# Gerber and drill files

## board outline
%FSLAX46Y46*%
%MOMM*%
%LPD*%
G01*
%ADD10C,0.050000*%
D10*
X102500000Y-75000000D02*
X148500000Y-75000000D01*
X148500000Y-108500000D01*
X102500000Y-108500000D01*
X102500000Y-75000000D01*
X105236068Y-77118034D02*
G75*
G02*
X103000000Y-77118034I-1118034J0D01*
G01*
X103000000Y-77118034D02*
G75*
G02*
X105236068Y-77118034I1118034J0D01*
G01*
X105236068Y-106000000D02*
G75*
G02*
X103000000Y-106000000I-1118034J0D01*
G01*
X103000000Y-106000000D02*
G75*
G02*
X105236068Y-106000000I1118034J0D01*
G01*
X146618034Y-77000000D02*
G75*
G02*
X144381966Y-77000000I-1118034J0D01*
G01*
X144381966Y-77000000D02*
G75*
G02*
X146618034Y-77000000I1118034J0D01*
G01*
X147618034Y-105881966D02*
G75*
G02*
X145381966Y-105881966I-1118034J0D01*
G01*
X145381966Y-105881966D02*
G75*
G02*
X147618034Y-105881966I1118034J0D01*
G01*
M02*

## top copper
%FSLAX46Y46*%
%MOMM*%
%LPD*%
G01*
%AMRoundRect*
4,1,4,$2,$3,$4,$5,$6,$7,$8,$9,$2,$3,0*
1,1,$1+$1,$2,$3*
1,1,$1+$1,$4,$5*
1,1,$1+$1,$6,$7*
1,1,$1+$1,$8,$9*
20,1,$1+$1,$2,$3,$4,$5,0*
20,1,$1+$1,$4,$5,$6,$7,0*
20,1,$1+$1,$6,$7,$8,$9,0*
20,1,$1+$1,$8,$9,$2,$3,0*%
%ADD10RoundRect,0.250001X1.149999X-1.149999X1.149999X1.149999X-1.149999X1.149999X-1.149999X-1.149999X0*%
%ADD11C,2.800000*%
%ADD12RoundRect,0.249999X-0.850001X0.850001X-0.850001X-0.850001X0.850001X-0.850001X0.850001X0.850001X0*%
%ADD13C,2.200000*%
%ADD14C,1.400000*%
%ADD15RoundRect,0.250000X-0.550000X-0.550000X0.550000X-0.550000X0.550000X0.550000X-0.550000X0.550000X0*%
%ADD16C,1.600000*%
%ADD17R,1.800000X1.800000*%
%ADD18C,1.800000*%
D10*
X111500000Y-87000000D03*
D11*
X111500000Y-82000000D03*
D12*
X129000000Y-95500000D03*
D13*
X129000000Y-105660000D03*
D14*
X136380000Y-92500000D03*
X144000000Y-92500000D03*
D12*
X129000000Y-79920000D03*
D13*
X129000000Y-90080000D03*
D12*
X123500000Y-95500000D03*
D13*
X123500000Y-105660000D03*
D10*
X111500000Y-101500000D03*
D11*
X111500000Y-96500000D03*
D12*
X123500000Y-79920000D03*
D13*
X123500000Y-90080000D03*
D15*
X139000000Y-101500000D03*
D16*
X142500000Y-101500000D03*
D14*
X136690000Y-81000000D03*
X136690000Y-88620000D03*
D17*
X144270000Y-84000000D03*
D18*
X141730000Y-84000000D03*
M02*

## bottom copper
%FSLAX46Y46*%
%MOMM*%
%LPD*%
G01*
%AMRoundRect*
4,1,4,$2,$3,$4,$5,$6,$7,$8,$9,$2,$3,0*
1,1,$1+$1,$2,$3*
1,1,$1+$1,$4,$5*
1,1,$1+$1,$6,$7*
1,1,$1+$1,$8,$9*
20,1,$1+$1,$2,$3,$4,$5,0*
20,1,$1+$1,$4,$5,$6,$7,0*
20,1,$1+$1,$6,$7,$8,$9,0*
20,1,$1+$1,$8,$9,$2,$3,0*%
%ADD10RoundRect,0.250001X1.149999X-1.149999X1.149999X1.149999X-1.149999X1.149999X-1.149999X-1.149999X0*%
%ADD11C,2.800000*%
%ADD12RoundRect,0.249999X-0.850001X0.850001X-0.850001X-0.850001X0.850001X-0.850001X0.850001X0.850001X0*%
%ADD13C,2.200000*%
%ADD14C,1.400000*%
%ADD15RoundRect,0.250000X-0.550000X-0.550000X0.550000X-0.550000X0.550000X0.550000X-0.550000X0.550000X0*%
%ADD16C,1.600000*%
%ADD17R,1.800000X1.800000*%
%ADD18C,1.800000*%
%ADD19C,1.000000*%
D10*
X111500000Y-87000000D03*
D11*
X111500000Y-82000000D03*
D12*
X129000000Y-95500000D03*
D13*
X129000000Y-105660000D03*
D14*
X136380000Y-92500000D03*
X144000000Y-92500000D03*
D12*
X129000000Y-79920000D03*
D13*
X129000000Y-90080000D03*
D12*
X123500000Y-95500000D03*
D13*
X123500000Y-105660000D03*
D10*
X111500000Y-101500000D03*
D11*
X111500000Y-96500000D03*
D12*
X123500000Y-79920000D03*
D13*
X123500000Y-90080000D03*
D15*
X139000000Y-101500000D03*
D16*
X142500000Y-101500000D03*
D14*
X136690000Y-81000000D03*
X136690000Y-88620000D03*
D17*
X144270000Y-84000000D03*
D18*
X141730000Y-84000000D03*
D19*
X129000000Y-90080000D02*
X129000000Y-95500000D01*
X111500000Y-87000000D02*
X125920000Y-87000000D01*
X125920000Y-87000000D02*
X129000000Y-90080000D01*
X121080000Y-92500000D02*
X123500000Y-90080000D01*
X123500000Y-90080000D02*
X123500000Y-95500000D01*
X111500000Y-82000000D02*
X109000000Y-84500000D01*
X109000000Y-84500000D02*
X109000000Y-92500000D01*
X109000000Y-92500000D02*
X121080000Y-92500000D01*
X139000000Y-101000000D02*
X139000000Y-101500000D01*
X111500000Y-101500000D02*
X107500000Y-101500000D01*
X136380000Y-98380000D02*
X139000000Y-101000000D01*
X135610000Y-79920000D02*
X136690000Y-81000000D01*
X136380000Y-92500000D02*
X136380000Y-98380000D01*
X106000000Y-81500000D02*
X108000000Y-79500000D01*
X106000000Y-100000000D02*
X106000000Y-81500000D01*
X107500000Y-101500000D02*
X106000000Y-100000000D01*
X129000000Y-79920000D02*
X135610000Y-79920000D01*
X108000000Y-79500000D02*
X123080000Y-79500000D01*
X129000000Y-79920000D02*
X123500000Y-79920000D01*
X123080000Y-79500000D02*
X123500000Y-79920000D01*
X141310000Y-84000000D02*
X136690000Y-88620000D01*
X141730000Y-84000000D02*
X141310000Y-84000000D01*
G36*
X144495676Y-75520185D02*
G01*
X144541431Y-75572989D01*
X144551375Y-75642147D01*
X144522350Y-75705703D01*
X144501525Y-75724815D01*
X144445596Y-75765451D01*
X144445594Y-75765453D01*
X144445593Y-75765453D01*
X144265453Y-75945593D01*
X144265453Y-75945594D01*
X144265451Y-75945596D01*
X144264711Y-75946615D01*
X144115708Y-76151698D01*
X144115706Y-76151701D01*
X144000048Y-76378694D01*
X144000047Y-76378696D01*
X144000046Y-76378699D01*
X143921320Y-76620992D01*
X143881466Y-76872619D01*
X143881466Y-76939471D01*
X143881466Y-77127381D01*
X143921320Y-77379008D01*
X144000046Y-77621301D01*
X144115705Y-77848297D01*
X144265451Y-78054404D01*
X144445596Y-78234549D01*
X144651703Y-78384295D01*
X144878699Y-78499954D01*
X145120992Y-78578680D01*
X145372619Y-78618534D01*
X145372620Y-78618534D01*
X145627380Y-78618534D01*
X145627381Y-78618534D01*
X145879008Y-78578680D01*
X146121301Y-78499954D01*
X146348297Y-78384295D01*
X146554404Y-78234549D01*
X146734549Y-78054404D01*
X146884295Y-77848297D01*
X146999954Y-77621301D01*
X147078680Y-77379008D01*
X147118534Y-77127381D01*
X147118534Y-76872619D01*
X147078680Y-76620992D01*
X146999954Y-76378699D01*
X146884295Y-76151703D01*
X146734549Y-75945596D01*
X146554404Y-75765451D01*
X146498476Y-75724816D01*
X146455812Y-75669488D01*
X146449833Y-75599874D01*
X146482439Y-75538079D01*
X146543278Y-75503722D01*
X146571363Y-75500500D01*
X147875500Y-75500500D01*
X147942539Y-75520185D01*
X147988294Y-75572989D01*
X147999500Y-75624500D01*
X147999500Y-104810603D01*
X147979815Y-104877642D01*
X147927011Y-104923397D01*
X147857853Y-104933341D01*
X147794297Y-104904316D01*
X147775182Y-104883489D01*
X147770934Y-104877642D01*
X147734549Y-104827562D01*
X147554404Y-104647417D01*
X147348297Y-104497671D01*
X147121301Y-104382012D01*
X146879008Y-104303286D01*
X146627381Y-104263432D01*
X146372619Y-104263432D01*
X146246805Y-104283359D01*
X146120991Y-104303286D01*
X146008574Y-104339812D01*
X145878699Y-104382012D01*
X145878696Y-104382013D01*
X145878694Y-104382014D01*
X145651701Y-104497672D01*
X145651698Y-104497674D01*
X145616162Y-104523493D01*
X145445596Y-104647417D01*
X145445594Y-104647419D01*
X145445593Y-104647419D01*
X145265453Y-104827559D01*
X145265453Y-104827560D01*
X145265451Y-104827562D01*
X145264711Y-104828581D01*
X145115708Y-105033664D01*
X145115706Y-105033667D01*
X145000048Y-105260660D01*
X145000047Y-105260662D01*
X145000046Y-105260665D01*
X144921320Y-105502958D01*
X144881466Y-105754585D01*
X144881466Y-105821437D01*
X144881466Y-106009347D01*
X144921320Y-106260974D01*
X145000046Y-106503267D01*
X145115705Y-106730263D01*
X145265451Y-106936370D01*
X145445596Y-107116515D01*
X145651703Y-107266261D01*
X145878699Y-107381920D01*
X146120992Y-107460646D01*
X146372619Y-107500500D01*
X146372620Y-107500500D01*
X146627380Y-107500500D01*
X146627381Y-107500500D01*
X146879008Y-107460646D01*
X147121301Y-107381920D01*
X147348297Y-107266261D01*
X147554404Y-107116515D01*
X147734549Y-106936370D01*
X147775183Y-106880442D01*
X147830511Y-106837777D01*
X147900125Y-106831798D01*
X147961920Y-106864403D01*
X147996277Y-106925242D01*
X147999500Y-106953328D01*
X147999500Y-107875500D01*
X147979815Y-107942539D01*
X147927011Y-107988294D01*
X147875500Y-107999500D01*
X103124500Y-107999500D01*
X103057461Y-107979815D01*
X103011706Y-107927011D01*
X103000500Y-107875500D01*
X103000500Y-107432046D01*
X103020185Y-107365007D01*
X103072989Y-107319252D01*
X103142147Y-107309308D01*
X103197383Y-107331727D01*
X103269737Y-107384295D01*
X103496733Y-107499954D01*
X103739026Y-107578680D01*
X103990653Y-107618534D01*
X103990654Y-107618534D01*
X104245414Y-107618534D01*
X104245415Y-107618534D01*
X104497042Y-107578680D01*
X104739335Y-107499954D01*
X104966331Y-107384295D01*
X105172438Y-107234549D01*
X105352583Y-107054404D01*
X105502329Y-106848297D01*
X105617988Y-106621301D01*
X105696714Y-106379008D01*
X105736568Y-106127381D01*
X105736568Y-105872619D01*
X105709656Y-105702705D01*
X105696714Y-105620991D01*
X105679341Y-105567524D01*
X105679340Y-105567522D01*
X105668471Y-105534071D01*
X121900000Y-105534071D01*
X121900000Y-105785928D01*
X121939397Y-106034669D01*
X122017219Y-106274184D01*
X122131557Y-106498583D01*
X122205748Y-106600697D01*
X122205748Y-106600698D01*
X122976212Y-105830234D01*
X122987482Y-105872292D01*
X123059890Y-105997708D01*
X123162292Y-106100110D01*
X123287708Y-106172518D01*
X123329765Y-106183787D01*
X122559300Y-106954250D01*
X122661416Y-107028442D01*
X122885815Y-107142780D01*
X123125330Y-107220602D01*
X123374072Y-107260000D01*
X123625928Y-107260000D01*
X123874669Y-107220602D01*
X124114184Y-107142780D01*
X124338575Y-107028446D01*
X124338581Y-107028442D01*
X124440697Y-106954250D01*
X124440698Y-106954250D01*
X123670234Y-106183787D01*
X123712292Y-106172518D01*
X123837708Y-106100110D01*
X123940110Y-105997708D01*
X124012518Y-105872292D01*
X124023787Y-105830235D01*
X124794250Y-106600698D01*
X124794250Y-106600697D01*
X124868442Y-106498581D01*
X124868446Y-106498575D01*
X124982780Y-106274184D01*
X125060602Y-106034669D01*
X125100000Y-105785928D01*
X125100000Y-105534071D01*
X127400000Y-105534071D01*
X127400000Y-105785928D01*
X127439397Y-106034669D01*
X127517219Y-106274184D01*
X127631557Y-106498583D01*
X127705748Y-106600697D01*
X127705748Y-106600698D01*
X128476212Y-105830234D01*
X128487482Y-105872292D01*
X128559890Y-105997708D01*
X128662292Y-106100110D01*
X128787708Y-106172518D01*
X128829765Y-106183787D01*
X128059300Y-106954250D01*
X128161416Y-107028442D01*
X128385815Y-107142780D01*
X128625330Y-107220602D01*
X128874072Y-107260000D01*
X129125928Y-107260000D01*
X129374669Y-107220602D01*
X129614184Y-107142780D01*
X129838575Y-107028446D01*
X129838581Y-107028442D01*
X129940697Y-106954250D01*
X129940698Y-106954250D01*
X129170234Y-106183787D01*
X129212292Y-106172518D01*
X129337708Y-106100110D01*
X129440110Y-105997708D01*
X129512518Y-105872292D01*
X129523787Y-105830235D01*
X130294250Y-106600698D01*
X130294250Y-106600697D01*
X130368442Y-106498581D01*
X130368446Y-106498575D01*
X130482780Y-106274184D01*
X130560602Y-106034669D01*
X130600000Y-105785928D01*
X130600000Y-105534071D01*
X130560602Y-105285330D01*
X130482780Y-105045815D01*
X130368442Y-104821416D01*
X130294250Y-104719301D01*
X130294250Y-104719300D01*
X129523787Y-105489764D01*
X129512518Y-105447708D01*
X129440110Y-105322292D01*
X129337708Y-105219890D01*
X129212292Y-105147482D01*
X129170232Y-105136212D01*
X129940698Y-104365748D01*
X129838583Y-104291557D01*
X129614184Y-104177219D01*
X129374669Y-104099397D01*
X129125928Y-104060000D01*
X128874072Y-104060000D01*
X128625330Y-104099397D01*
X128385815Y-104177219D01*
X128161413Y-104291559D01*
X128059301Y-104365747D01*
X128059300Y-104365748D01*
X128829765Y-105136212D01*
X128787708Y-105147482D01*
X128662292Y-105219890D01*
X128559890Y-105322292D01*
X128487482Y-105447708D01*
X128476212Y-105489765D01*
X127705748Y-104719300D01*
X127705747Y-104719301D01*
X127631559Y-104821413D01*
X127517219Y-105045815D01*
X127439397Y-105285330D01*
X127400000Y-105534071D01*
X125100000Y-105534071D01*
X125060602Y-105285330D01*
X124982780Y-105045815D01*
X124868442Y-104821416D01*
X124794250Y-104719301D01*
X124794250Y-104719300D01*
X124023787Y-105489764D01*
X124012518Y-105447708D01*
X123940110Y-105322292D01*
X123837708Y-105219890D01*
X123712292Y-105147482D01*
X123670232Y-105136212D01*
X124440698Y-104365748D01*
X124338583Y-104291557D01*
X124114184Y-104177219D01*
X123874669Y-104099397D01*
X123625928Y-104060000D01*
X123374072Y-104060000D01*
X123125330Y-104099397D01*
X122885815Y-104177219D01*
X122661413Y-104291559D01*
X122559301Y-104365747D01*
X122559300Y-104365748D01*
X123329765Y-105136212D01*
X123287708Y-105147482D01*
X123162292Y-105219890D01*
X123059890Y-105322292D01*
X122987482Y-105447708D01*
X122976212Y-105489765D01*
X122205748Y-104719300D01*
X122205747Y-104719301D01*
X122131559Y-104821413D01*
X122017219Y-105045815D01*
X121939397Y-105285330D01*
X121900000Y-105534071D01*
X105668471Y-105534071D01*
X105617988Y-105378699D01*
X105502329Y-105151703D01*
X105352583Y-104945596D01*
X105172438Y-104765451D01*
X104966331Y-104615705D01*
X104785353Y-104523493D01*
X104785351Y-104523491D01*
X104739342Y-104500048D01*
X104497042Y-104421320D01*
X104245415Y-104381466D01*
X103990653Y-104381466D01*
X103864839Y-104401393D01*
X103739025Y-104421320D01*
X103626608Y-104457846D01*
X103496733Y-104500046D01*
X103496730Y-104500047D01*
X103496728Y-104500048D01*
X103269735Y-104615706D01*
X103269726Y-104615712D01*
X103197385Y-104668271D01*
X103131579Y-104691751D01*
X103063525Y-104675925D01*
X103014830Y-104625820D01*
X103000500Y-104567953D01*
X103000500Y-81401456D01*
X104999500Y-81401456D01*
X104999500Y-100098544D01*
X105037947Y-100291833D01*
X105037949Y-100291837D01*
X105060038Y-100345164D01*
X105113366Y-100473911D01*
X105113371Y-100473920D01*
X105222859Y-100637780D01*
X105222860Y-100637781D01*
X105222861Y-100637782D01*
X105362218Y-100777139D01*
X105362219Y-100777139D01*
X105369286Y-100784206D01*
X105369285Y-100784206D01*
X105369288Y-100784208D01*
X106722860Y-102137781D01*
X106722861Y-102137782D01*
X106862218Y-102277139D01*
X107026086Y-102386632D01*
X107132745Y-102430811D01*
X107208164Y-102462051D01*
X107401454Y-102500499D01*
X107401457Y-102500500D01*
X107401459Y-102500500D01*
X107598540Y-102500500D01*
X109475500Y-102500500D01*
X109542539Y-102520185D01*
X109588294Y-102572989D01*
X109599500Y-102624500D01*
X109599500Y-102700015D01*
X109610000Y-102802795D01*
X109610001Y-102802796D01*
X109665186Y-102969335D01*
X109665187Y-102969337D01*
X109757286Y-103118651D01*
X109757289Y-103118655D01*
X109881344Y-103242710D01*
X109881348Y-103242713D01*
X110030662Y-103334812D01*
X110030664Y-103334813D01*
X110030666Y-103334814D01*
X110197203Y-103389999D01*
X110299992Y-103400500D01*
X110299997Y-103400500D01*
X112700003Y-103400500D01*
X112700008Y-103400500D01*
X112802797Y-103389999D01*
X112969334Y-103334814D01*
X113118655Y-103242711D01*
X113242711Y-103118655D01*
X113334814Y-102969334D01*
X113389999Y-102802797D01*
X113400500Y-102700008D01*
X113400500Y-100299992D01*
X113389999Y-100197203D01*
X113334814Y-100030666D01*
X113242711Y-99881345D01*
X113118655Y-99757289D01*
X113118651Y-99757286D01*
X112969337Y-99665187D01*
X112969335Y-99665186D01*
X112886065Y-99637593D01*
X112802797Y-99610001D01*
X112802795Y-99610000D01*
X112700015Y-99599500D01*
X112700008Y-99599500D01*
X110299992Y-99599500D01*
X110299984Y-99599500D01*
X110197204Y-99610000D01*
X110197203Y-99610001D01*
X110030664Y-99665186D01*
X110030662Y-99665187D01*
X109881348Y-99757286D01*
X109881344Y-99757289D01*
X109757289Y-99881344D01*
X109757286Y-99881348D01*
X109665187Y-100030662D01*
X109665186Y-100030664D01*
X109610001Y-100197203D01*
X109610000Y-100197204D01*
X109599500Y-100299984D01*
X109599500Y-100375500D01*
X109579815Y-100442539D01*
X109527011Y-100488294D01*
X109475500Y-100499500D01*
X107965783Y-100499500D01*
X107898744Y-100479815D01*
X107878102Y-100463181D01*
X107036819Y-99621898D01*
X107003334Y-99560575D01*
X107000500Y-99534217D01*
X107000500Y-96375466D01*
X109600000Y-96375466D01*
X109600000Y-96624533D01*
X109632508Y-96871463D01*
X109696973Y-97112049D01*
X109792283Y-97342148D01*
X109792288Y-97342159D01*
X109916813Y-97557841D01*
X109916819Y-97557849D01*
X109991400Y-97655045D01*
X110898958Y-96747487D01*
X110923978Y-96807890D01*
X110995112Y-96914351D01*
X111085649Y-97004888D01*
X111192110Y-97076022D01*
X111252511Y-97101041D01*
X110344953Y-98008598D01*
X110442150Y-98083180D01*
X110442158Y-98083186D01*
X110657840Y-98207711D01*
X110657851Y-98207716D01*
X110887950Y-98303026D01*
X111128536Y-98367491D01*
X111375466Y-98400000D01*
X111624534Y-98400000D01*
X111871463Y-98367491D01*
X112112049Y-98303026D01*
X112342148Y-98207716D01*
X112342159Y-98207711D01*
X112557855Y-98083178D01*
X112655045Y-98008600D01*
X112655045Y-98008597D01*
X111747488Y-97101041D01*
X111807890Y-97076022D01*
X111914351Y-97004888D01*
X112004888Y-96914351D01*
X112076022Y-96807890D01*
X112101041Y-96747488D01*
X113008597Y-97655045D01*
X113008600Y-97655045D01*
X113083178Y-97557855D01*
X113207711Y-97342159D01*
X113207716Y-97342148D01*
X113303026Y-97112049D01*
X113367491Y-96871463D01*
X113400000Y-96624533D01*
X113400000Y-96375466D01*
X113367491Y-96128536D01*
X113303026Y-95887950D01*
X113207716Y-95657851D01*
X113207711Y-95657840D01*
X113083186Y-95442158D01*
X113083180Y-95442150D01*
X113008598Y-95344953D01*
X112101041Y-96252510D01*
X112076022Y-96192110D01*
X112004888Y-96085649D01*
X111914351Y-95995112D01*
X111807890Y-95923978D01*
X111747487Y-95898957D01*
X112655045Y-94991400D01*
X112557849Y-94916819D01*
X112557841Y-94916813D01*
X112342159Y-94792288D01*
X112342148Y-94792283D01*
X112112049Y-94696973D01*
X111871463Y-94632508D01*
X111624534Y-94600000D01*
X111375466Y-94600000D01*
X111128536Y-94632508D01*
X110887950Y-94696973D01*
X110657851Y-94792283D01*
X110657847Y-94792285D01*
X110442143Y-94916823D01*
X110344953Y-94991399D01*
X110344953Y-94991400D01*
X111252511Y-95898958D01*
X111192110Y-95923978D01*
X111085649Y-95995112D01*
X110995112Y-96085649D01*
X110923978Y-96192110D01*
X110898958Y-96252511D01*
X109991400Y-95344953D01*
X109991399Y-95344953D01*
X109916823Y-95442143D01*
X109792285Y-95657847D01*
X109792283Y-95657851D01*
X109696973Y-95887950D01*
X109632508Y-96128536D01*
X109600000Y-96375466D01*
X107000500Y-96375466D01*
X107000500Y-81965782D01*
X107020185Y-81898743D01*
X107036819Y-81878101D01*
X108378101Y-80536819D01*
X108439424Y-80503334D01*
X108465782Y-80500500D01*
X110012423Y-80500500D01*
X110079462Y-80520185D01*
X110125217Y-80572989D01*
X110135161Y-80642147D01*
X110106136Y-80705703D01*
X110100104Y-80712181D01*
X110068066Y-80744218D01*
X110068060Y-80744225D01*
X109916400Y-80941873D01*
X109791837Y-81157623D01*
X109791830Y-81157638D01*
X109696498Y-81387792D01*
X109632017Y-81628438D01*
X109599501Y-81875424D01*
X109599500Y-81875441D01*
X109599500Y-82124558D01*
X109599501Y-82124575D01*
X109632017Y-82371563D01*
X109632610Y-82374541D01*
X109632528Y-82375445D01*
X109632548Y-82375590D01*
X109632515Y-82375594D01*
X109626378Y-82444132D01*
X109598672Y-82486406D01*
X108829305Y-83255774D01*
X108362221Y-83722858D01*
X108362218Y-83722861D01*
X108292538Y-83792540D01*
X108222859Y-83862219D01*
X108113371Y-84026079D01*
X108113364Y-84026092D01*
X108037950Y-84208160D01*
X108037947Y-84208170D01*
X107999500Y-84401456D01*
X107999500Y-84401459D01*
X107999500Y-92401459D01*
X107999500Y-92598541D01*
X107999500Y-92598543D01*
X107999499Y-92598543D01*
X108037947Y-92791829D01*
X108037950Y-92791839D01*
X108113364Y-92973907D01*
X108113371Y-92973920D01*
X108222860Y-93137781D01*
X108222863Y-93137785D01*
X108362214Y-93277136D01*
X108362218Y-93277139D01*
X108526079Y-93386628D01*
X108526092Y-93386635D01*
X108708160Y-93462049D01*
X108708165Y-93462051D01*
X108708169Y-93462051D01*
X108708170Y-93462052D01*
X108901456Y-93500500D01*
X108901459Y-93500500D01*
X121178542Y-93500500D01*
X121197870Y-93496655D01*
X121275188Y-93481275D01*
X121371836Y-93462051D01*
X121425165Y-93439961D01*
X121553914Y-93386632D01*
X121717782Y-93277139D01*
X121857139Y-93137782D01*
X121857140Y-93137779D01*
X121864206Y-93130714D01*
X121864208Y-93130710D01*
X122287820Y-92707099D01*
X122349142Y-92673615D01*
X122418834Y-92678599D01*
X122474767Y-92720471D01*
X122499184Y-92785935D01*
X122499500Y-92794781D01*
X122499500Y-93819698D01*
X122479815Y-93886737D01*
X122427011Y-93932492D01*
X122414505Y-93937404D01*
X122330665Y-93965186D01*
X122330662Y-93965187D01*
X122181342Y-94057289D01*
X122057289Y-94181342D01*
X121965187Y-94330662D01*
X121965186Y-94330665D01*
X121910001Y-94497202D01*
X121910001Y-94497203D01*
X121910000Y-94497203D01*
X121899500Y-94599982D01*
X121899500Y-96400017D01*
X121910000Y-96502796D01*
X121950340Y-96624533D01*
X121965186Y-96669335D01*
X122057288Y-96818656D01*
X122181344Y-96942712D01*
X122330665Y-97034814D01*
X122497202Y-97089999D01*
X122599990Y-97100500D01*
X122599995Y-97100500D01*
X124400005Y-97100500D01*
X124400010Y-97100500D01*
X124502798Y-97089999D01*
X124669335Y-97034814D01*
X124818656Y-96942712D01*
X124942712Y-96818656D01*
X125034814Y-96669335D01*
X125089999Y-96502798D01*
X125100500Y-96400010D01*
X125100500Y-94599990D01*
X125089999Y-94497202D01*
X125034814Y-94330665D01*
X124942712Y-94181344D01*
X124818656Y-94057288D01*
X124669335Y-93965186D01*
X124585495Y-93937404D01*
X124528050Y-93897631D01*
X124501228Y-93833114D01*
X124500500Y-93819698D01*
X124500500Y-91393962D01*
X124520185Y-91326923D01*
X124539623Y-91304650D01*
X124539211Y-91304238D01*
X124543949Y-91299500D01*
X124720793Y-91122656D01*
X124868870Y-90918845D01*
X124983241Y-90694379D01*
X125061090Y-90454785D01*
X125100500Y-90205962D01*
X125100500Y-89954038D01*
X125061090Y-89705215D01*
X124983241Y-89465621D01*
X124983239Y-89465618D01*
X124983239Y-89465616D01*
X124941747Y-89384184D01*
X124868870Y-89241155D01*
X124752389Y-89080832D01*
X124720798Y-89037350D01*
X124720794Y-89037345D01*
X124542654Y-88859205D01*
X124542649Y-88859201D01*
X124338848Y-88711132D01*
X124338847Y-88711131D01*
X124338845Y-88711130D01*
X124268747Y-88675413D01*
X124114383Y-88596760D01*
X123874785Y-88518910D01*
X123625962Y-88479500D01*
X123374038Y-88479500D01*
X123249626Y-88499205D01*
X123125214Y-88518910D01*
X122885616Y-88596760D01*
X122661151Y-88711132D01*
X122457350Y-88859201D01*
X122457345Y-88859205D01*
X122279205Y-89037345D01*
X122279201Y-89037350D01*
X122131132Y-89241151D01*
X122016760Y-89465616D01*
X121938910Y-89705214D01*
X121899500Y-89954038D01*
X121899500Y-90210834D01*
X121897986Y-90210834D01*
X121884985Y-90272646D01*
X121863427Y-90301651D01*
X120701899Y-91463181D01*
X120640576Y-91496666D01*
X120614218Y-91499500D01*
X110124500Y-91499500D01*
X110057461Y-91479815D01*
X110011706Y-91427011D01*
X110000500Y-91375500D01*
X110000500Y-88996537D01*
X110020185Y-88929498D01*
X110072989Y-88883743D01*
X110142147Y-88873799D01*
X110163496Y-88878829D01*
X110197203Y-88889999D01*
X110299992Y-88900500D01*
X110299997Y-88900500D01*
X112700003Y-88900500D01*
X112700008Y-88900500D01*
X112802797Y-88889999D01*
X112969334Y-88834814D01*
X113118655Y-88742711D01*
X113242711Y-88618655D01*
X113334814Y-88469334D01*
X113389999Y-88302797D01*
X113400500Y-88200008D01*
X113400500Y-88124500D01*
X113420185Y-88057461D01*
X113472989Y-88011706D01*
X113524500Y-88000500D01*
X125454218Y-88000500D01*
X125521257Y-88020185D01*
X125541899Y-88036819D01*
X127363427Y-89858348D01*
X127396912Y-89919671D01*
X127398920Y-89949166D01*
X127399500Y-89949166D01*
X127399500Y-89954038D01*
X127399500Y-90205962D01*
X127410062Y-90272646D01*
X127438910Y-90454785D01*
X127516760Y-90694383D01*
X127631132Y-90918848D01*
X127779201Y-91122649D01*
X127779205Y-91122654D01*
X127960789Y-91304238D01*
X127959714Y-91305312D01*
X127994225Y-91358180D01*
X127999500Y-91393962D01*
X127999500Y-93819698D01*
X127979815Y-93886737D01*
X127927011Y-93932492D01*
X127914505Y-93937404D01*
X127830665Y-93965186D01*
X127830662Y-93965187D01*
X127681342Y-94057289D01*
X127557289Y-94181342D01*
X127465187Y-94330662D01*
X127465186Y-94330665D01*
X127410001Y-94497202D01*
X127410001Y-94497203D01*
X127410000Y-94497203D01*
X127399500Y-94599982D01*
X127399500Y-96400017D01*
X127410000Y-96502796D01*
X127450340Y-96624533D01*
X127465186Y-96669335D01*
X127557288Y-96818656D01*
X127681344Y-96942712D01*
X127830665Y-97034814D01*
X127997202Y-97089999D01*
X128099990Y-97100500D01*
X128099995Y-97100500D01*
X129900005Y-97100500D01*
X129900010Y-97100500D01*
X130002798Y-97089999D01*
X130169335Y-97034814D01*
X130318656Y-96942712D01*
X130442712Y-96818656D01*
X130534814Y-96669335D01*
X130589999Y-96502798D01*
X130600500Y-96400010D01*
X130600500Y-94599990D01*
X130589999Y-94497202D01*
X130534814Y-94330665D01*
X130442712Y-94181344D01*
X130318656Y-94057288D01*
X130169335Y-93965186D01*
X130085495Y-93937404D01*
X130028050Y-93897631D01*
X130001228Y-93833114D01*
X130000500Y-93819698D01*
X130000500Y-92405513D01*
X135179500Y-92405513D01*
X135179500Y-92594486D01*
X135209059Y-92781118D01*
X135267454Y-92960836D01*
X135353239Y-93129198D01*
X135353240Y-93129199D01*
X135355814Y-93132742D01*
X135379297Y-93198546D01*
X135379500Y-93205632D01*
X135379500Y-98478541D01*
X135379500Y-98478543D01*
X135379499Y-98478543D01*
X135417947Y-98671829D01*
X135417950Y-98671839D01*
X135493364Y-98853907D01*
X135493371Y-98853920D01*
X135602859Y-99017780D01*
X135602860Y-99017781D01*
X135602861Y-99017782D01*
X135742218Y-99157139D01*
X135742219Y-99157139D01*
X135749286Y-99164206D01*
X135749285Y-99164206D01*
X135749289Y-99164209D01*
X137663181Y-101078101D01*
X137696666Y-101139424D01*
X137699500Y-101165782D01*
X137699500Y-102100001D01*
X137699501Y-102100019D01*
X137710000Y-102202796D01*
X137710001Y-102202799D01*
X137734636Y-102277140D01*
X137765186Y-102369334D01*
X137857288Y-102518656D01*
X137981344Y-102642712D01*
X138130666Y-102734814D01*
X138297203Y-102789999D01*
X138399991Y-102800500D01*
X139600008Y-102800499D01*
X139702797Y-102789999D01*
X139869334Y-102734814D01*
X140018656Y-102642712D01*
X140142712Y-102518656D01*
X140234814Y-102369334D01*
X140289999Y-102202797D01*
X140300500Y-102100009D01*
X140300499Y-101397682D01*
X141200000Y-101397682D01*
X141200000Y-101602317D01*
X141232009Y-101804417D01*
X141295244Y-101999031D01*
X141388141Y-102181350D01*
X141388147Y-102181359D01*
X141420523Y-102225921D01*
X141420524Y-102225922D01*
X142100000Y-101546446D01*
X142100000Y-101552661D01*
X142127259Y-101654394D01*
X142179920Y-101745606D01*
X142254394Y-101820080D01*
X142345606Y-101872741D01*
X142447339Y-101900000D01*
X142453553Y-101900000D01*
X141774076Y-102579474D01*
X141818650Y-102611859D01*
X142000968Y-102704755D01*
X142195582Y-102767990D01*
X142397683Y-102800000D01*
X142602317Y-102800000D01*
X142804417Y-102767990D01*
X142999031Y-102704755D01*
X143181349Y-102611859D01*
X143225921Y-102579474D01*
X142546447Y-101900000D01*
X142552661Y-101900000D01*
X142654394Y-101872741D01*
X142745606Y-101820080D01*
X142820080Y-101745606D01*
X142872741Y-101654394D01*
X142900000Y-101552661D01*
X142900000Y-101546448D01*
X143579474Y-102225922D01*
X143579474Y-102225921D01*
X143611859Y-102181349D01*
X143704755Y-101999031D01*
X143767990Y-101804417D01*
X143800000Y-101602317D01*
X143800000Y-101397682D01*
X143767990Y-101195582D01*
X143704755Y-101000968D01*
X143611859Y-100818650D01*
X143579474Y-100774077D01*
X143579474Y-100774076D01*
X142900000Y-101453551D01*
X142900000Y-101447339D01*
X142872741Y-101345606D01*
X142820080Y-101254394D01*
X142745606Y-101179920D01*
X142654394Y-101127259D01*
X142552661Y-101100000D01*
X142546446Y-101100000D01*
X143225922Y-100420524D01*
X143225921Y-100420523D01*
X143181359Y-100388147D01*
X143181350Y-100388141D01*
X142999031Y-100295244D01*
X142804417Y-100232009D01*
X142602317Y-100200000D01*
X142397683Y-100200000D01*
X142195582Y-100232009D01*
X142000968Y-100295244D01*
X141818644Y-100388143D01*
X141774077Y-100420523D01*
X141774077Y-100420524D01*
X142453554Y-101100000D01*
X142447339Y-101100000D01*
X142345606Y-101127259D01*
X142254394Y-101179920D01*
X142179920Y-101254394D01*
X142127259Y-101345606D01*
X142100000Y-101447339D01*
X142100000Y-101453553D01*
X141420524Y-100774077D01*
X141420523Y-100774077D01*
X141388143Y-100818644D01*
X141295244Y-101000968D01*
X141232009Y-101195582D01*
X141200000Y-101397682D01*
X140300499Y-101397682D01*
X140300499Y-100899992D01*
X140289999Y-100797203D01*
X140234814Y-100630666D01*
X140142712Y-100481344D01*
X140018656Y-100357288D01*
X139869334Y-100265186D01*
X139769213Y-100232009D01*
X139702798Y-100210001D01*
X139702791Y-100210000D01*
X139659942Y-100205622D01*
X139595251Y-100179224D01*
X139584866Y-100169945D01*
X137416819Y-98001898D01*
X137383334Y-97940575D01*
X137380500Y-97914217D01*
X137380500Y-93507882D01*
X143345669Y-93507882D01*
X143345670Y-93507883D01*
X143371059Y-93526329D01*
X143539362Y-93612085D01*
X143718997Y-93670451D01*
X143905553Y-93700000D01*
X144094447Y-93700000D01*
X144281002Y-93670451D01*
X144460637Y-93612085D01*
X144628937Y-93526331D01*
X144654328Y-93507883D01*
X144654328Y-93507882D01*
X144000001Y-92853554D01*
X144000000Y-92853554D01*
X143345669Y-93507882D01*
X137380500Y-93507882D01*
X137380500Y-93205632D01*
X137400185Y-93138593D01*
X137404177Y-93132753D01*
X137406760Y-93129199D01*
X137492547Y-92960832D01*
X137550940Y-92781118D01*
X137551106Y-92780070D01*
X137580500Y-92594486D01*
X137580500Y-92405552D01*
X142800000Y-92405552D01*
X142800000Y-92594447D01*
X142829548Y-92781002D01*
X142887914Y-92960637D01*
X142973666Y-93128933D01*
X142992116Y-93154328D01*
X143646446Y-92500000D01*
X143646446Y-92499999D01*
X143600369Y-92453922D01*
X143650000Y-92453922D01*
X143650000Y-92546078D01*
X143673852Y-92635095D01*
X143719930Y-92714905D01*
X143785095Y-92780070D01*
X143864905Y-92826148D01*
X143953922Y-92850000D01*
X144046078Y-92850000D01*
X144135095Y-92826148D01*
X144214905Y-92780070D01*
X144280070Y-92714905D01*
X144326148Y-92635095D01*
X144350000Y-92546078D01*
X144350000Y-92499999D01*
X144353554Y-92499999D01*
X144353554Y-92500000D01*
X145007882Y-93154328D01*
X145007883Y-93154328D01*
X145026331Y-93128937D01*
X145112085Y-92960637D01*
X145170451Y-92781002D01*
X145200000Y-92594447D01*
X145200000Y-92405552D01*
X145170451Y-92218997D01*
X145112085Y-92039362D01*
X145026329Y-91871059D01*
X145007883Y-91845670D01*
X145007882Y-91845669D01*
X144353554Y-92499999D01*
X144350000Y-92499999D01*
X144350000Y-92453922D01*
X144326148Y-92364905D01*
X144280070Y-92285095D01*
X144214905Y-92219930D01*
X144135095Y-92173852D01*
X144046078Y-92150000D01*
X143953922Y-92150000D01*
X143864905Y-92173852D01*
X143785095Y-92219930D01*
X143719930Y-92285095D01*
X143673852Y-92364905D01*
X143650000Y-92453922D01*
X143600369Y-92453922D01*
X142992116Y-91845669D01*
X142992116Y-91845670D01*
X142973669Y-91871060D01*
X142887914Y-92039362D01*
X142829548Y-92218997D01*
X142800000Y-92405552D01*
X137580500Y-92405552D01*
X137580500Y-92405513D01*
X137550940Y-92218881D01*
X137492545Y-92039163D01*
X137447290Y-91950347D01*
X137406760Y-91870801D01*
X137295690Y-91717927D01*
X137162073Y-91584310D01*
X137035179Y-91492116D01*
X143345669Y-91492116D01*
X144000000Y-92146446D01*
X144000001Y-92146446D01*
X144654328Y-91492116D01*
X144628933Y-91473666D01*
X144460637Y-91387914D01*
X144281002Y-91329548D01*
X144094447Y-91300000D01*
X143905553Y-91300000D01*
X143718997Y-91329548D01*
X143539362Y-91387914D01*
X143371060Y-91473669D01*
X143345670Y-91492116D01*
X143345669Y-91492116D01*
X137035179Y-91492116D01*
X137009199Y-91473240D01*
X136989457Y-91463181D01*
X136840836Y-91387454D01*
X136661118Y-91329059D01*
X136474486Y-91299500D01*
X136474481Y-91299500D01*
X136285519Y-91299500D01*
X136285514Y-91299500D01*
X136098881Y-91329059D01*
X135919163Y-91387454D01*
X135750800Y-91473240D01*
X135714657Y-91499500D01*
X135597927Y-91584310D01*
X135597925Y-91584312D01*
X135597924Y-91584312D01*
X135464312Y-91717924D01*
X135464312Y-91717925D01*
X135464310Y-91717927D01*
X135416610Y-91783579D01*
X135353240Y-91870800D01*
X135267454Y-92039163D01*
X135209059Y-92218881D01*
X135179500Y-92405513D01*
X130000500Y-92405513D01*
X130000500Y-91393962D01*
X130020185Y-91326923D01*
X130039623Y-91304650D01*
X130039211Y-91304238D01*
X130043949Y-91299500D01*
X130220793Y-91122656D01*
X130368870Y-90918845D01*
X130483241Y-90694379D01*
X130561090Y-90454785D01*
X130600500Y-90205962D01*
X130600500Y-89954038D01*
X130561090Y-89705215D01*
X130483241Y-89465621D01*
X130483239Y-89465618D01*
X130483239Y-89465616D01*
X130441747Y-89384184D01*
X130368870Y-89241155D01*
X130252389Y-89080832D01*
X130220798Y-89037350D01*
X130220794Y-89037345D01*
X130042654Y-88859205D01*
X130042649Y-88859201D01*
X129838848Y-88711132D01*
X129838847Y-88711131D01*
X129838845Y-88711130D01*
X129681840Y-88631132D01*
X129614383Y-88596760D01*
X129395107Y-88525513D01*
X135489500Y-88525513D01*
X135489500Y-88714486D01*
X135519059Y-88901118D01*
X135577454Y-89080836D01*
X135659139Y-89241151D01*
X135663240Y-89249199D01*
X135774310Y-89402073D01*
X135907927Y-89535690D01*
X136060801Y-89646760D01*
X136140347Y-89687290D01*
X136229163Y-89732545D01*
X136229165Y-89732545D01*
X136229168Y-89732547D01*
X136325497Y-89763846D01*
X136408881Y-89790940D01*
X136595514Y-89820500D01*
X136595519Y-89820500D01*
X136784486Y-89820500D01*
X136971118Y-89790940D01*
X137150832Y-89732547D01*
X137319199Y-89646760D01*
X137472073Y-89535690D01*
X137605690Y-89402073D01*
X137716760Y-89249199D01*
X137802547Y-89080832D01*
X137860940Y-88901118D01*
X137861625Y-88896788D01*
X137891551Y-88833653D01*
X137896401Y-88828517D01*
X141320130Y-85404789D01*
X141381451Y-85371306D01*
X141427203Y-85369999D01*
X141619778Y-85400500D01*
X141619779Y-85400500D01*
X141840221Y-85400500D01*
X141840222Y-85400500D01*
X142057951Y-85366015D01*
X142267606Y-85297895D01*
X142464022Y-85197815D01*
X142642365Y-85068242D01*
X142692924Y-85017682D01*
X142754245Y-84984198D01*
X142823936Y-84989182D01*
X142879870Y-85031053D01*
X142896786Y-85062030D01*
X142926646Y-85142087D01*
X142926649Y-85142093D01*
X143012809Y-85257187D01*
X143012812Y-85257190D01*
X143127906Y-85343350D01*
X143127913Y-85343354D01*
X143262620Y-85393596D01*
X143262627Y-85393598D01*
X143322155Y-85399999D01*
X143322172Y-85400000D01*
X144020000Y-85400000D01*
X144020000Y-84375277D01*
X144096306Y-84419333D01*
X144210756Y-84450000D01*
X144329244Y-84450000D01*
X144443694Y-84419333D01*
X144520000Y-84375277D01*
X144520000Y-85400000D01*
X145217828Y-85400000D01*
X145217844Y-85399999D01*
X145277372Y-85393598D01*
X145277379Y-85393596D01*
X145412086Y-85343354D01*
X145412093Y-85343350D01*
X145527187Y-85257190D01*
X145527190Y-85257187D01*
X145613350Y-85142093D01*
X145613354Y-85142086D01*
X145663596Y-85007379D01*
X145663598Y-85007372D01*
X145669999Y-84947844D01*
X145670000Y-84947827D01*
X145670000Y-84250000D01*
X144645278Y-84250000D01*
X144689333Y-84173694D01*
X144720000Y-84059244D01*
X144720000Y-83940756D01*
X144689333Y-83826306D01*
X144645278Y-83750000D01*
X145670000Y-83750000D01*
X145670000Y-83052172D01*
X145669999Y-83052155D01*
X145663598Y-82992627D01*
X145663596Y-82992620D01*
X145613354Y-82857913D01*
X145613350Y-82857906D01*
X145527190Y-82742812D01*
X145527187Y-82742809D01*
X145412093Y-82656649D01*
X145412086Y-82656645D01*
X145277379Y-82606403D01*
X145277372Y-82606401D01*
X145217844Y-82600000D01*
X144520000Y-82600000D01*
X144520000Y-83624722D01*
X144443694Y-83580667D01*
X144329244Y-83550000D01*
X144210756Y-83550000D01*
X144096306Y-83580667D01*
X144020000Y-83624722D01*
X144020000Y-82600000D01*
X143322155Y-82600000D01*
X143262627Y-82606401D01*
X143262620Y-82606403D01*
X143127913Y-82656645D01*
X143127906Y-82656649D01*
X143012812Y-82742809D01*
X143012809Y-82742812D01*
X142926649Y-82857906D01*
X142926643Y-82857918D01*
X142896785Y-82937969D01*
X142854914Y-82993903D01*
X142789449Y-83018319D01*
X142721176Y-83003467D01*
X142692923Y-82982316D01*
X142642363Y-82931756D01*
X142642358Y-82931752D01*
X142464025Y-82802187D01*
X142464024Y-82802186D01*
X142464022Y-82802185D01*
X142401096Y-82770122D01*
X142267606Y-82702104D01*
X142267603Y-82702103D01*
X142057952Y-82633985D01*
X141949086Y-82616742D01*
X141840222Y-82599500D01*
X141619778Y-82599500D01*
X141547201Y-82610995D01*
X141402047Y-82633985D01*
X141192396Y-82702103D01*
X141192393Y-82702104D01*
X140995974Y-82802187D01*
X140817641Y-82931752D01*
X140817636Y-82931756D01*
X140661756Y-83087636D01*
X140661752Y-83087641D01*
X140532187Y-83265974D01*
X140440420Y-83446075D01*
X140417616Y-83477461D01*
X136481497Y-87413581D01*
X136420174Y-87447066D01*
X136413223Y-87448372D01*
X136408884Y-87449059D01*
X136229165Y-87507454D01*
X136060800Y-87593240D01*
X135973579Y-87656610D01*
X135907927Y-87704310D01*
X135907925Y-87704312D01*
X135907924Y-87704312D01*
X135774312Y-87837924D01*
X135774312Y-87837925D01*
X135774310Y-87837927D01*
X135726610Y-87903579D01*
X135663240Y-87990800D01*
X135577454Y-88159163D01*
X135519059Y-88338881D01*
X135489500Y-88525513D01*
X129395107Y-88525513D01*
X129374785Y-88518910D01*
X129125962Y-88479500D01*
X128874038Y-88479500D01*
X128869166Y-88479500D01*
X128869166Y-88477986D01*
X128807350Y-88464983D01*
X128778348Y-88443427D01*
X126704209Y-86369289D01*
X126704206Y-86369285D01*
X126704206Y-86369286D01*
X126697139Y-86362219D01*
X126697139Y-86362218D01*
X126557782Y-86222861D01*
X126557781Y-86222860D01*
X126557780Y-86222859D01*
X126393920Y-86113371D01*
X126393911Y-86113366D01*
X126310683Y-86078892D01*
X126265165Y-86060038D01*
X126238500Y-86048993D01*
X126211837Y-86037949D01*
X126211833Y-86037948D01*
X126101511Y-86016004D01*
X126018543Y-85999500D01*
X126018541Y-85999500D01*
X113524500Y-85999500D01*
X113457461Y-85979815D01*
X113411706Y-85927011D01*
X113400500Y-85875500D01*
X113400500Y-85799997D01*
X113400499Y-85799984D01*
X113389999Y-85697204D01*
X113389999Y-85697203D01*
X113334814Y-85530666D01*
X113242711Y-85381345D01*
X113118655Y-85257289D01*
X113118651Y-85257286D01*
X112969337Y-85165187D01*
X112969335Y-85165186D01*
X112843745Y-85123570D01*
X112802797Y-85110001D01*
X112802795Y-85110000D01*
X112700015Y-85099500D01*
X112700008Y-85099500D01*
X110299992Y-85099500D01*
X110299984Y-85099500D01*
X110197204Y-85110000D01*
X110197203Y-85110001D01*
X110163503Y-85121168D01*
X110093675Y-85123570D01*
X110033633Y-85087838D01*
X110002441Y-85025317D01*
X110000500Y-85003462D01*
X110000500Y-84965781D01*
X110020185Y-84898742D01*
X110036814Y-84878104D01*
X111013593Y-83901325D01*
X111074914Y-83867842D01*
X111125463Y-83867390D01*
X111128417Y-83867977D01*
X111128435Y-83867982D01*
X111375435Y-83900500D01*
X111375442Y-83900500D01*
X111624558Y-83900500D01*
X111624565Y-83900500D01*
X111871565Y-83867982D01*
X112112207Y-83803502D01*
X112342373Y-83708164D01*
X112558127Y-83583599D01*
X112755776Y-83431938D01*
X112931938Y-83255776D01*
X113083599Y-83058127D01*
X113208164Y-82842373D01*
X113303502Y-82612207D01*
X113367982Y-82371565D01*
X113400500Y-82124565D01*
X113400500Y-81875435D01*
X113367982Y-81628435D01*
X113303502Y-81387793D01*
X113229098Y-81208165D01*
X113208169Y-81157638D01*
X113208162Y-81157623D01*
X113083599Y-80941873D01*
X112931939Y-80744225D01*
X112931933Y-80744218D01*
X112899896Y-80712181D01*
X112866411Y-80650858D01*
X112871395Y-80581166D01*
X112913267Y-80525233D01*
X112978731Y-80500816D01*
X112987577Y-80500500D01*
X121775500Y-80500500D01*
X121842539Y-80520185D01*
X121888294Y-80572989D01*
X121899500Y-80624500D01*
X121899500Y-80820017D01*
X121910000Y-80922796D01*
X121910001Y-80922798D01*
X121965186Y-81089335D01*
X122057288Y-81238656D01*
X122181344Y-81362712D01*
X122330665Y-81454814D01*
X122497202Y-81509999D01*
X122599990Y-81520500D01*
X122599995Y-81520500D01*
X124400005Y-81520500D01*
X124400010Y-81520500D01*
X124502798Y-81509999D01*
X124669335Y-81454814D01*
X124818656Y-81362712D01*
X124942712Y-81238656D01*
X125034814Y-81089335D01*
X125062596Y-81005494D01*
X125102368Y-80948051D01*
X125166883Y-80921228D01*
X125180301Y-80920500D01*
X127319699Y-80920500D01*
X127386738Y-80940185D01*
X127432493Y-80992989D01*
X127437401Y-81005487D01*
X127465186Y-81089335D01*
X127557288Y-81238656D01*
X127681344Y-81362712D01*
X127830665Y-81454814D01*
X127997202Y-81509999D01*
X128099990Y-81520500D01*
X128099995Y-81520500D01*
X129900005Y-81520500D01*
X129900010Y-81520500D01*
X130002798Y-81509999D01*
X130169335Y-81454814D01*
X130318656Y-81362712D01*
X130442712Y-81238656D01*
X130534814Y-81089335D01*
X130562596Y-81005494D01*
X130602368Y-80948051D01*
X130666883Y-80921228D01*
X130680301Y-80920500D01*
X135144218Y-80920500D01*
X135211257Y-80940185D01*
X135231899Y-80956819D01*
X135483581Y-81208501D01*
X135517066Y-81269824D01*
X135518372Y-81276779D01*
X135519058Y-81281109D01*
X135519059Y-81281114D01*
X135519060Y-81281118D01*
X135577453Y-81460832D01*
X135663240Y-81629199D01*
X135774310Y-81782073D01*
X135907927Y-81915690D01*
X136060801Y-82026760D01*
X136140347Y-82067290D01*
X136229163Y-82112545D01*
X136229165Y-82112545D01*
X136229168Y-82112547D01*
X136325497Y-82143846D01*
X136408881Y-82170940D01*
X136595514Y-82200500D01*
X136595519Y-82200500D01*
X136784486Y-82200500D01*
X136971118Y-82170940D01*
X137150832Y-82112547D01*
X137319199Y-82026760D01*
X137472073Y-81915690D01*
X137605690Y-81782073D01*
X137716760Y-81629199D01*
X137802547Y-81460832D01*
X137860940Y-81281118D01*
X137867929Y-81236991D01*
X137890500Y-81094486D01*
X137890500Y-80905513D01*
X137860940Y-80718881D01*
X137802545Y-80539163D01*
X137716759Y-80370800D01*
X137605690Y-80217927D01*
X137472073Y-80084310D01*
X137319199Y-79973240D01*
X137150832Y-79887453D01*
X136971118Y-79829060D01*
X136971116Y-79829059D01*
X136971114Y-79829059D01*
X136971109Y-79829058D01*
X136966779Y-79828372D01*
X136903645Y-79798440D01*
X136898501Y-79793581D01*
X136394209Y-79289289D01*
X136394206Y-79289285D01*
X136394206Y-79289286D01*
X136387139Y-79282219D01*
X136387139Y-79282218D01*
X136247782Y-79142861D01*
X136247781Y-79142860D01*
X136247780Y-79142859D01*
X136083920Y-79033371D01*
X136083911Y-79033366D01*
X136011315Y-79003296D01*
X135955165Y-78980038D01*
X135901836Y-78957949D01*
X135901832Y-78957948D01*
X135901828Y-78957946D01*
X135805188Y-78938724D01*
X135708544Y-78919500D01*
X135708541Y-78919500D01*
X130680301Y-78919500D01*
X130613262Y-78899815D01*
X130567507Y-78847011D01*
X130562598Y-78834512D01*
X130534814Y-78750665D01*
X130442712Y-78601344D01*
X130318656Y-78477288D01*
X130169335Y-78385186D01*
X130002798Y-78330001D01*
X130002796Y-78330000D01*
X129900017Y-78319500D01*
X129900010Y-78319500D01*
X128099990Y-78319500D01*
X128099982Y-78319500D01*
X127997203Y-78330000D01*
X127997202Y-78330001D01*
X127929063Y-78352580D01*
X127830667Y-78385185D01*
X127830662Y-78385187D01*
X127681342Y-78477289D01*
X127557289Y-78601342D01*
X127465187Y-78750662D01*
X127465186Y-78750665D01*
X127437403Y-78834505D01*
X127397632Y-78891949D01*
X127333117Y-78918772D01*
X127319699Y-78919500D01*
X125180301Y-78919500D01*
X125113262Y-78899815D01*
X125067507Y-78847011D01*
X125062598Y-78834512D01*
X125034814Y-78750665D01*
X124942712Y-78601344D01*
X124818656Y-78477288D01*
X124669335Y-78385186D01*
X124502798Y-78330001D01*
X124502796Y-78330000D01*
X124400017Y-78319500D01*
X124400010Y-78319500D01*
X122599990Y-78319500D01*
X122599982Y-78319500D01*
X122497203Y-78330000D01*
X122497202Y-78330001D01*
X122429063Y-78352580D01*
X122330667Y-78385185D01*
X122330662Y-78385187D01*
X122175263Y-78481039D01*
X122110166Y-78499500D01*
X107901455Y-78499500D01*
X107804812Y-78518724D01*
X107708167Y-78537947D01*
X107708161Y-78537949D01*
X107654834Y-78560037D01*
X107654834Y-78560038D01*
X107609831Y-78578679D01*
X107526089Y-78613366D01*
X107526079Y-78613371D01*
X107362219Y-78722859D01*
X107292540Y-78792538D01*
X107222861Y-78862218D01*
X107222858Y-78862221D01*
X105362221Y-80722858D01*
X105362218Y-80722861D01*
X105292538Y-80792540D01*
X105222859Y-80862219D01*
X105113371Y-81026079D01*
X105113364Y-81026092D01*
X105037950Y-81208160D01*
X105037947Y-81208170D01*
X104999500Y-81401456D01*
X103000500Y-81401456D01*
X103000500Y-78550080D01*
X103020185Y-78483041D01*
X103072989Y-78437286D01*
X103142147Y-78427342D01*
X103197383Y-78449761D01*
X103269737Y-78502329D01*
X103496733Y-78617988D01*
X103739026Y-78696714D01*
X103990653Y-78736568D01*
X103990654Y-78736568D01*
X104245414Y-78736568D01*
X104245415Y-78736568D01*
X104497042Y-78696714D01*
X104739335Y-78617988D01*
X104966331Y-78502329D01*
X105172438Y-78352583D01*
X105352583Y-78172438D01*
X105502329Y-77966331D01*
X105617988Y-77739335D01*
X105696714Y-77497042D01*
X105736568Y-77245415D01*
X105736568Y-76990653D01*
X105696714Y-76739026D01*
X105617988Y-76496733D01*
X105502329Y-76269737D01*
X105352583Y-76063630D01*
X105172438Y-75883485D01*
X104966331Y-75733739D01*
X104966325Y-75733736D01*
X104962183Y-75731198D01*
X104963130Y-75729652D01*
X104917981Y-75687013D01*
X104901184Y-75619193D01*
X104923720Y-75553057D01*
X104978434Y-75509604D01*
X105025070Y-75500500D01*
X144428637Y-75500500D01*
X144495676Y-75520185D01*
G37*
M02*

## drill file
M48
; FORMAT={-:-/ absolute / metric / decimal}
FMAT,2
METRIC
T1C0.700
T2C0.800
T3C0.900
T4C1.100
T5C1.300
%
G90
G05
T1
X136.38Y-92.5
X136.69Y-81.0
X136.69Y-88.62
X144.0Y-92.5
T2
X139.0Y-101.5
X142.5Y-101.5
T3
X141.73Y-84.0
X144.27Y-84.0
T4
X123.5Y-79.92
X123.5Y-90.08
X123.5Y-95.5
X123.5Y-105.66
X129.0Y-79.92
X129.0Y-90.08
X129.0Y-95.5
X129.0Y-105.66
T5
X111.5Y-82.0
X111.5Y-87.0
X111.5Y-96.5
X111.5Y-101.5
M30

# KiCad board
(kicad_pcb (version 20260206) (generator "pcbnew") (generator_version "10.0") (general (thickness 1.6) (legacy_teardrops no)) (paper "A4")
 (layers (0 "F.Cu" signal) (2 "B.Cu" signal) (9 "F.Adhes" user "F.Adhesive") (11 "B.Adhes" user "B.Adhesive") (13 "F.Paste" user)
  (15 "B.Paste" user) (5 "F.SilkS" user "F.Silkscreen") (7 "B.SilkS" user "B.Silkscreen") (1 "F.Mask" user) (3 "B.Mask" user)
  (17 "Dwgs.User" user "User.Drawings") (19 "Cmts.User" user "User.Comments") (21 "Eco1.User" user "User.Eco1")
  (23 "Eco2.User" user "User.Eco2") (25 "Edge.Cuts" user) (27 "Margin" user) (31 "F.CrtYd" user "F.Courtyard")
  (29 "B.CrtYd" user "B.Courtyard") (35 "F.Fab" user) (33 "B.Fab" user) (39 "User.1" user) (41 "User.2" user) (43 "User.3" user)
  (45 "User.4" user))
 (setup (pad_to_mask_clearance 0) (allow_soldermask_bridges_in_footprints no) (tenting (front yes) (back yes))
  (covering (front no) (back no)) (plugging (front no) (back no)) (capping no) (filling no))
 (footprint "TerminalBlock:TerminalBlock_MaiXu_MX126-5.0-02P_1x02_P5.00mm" (layer "F.Cu") (at 111.5 87 90)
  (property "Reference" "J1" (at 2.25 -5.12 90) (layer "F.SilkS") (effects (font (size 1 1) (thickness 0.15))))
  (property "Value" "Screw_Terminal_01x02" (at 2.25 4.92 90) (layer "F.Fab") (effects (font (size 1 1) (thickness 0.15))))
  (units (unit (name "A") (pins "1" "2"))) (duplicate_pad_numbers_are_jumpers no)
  (pad "1" thru_hole roundrect (at 0 0 90) (size 2.8 2.8) (drill 1.3) (layers "*.Cu" "*.Mask") (remove_unused_layers no)
   (roundrect_rratio 0.089286) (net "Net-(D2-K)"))
  (pad "2" thru_hole circle (at 5 0 90) (size 2.8 2.8) (drill 1.3) (layers "*.Cu" "*.Mask") (remove_unused_layers no) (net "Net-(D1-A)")))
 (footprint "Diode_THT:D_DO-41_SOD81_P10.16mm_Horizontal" (layer "F.Cu") (at 129 95.5 -90)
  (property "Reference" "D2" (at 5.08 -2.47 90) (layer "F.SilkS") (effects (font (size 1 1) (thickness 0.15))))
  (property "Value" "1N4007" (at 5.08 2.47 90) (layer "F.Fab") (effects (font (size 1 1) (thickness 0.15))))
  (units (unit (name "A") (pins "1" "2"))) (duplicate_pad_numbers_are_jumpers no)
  (pad "1" thru_hole roundrect (at 0 0 270) (size 2.2 2.2) (drill 1.1) (layers "*.Cu" "*.Mask") (remove_unused_layers no)
   (roundrect_rratio 0.113636) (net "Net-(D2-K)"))
  (pad "2" thru_hole circle (at 10.16 0 270) (size 2.2 2.2) (drill 1.1) (layers "*.Cu" "*.Mask") (remove_unused_layers no) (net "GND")))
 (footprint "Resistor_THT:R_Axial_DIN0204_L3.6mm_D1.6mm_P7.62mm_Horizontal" (layer "F.Cu") (at 136.38 92.5)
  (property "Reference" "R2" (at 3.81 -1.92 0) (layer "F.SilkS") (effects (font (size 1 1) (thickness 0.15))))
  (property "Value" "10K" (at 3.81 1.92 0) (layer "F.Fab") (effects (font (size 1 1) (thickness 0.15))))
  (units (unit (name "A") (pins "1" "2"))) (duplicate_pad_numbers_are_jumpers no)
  (pad "1" thru_hole circle (at 0 0) (size 1.4 1.4) (drill 0.7) (layers "*.Cu" "*.Mask") (remove_unused_layers no) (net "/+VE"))
  (pad "2" thru_hole circle (at 7.62 0) (size 1.4 1.4) (drill 0.7) (layers "*.Cu" "*.Mask") (remove_unused_layers no) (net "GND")))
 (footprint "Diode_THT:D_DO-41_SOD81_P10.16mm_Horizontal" (layer "F.Cu") (at 129 79.92 -90)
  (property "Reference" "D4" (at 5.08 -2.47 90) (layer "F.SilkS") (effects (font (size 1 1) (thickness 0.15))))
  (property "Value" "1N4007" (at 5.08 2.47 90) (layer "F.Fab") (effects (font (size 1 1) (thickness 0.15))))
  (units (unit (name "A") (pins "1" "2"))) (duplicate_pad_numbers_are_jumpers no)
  (pad "1" thru_hole roundrect (at 0 0 270) (size 2.2 2.2) (drill 1.1) (layers "*.Cu" "*.Mask") (remove_unused_layers no)
   (roundrect_rratio 0.113636) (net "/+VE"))
  (pad "2" thru_hole circle (at 10.16 0 270) (size 2.2 2.2) (drill 1.1) (layers "*.Cu" "*.Mask") (remove_unused_layers no)
   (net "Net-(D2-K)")))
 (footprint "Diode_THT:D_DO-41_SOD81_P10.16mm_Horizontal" (layer "F.Cu") (at 123.5 95.5 -90)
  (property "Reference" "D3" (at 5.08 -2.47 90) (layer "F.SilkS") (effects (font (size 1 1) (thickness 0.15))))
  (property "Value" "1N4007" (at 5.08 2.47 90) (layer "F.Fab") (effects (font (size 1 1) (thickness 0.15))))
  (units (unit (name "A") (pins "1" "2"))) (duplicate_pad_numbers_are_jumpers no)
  (pad "1" thru_hole roundrect (at 0 0 270) (size 2.2 2.2) (drill 1.1) (layers "*.Cu" "*.Mask") (remove_unused_layers no)
   (roundrect_rratio 0.113636) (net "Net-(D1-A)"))
  (pad "2" thru_hole circle (at 10.16 0 270) (size 2.2 2.2) (drill 1.1) (layers "*.Cu" "*.Mask") (remove_unused_layers no) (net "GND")))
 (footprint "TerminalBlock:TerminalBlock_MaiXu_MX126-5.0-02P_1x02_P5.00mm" (layer "F.Cu") (at 111.5 101.5 90)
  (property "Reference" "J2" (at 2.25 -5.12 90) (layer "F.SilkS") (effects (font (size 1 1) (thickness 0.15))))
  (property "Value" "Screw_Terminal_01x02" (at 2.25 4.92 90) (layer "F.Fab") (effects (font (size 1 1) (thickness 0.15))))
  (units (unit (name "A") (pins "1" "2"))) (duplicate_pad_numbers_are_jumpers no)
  (pad "1" thru_hole roundrect (at 0 0 90) (size 2.8 2.8) (drill 1.3) (layers "*.Cu" "*.Mask") (remove_unused_layers no)
   (roundrect_rratio 0.089286) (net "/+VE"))
  (pad "2" thru_hole circle (at 5 0 90) (size 2.8 2.8) (drill 1.3) (layers "*.Cu" "*.Mask") (remove_unused_layers no) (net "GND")))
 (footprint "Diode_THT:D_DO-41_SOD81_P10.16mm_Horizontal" (layer "F.Cu") (at 123.5 79.92 -90)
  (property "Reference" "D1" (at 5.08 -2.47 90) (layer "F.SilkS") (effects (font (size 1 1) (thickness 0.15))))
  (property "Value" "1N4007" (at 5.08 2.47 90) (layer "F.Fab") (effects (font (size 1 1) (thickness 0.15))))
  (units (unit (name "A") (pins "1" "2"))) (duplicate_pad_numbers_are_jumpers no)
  (pad "1" thru_hole roundrect (at 0 0 270) (size 2.2 2.2) (drill 1.1) (layers "*.Cu" "*.Mask") (remove_unused_layers no)
   (roundrect_rratio 0.113636) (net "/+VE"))
  (pad "2" thru_hole circle (at 10.16 0 270) (size 2.2 2.2) (drill 1.1) (layers "*.Cu" "*.Mask") (remove_unused_layers no)
   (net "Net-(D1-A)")))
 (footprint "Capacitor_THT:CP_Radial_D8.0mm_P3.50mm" (layer "F.Cu") (at 139 101.5)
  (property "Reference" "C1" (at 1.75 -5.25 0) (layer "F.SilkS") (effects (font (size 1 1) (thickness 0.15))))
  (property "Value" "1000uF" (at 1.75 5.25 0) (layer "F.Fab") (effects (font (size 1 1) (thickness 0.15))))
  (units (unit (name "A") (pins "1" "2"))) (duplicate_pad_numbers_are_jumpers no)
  (pad "1" thru_hole roundrect (at 0 0) (size 1.6 1.6) (drill 0.8) (layers "*.Cu" "*.Mask") (remove_unused_layers no)
   (roundrect_rratio 0.15625) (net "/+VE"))
  (pad "2" thru_hole circle (at 3.5 0) (size 1.6 1.6) (drill 0.8) (layers "*.Cu" "*.Mask") (remove_unused_layers no) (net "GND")))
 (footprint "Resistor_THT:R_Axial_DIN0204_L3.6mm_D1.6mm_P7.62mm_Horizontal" (layer "F.Cu") (at 136.69 81 -90)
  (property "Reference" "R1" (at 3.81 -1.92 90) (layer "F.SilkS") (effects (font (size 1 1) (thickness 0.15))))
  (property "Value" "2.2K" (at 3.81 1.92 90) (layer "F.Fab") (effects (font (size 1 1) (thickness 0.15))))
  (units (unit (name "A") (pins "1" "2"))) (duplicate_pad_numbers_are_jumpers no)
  (pad "1" thru_hole circle (at 0 0 270) (size 1.4 1.4) (drill 0.7) (layers "*.Cu" "*.Mask") (remove_unused_layers no) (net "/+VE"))
  (pad "2" thru_hole circle (at 7.62 0 270) (size 1.4 1.4) (drill 0.7) (layers "*.Cu" "*.Mask") (remove_unused_layers no) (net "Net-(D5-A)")))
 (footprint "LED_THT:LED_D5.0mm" (layer "F.Cu") (at 144.27 84 180)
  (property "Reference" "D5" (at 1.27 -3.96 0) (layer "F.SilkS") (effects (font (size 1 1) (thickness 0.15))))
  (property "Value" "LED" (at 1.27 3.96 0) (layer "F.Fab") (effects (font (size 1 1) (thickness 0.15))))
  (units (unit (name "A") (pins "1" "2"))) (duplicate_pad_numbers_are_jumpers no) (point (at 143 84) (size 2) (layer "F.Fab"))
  (pad "1" thru_hole rect (at 0 0 180) (size 1.8 1.8) (drill 0.9) (layers "*.Cu" "*.Mask") (remove_unused_layers no) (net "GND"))
  (pad "2" thru_hole circle (at 2.54 0 180) (size 1.8 1.8) (drill 0.9) (layers "*.Cu" "*.Mask") (remove_unused_layers no) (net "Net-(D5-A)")))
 (gr_rect (start 102.5 75) (end 148.5 108.5) (stroke (width 0.05) (type default)) (fill no) (layer "Edge.Cuts"))
 (gr_circle (center 104.118034 77.118034) (end 105.118034 77.618034) (stroke (width 0.05) (type default)) (fill no) (layer "Edge.Cuts"))
 (gr_circle (center 104.118034 106) (end 105.118034 106.5) (stroke (width 0.05) (type default)) (fill no) (layer "Edge.Cuts"))
 (gr_circle (center 145.5 77) (end 146.5 77.5) (stroke (width 0.05) (type default)) (fill no) (layer "Edge.Cuts"))
 (gr_circle (center 146.5 105.881966) (end 147.5 106.381966) (stroke (width 0.05) (type default)) (fill no) (layer "Edge.Cuts"))
 (segment (start 129 90.08) (end 129 95.5) (width 1) (layer "B.Cu") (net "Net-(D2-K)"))
 (segment (start 111.5 87) (end 125.92 87) (width 1) (layer "B.Cu") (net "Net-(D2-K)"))
 (segment (start 125.92 87) (end 129 90.08) (width 1) (layer "B.Cu") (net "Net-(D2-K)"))
 (segment (start 121.08 92.5) (end 123.5 90.08) (width 1) (layer "B.Cu") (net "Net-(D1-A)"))
 (segment (start 123.5 90.08) (end 123.5 95.5) (width 1) (layer "B.Cu") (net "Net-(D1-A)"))
 (segment (start 111.5 82) (end 109 84.5) (width 1) (layer "B.Cu") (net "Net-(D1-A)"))
 (segment (start 109 84.5) (end 109 92.5) (width 1) (layer "B.Cu") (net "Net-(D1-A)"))
 (segment (start 109 92.5) (end 121.08 92.5) (width 1) (layer "B.Cu") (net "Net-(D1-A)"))
 (segment (start 139 101) (end 139 101.5) (width 1) (layer "B.Cu") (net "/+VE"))
 (segment (start 111.5 101.5) (end 107.5 101.5) (width 1) (layer "B.Cu") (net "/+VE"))
 (segment (start 136.38 98.38) (end 139 101) (width 1) (layer "B.Cu") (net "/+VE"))
 (segment (start 135.61 79.92) (end 136.69 81) (width 1) (layer "B.Cu") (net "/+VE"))
 (segment (start 136.38 92.5) (end 136.38 98.38) (width 1) (layer "B.Cu") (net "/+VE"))
 (segment (start 106 81.5) (end 108 79.5) (width 1) (layer "B.Cu") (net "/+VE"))
 (segment (start 106 100) (end 106 81.5) (width 1) (layer "B.Cu") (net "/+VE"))
 (segment (start 107.5 101.5) (end 106 100) (width 1) (layer "B.Cu") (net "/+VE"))
 (segment (start 129 79.92) (end 135.61 79.92) (width 1) (layer "B.Cu") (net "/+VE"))
 (segment (start 108 79.5) (end 123.08 79.5) (width 1) (layer "B.Cu") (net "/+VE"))
 (segment (start 129 79.92) (end 123.5 79.92) (width 1) (layer "B.Cu") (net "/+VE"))
 (segment (start 123.08 79.5) (end 123.5 79.92) (width 1) (layer "B.Cu") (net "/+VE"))
 (segment (start 141.31 84) (end 136.69 88.62) (width 1) (layer "B.Cu") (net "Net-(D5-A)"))
 (segment (start 141.73 84) (end 141.31 84) (width 1) (layer "B.Cu") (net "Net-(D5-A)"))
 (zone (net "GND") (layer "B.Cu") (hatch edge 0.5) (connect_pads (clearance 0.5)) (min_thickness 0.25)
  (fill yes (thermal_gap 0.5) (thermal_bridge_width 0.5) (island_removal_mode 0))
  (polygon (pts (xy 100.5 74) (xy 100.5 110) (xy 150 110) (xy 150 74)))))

